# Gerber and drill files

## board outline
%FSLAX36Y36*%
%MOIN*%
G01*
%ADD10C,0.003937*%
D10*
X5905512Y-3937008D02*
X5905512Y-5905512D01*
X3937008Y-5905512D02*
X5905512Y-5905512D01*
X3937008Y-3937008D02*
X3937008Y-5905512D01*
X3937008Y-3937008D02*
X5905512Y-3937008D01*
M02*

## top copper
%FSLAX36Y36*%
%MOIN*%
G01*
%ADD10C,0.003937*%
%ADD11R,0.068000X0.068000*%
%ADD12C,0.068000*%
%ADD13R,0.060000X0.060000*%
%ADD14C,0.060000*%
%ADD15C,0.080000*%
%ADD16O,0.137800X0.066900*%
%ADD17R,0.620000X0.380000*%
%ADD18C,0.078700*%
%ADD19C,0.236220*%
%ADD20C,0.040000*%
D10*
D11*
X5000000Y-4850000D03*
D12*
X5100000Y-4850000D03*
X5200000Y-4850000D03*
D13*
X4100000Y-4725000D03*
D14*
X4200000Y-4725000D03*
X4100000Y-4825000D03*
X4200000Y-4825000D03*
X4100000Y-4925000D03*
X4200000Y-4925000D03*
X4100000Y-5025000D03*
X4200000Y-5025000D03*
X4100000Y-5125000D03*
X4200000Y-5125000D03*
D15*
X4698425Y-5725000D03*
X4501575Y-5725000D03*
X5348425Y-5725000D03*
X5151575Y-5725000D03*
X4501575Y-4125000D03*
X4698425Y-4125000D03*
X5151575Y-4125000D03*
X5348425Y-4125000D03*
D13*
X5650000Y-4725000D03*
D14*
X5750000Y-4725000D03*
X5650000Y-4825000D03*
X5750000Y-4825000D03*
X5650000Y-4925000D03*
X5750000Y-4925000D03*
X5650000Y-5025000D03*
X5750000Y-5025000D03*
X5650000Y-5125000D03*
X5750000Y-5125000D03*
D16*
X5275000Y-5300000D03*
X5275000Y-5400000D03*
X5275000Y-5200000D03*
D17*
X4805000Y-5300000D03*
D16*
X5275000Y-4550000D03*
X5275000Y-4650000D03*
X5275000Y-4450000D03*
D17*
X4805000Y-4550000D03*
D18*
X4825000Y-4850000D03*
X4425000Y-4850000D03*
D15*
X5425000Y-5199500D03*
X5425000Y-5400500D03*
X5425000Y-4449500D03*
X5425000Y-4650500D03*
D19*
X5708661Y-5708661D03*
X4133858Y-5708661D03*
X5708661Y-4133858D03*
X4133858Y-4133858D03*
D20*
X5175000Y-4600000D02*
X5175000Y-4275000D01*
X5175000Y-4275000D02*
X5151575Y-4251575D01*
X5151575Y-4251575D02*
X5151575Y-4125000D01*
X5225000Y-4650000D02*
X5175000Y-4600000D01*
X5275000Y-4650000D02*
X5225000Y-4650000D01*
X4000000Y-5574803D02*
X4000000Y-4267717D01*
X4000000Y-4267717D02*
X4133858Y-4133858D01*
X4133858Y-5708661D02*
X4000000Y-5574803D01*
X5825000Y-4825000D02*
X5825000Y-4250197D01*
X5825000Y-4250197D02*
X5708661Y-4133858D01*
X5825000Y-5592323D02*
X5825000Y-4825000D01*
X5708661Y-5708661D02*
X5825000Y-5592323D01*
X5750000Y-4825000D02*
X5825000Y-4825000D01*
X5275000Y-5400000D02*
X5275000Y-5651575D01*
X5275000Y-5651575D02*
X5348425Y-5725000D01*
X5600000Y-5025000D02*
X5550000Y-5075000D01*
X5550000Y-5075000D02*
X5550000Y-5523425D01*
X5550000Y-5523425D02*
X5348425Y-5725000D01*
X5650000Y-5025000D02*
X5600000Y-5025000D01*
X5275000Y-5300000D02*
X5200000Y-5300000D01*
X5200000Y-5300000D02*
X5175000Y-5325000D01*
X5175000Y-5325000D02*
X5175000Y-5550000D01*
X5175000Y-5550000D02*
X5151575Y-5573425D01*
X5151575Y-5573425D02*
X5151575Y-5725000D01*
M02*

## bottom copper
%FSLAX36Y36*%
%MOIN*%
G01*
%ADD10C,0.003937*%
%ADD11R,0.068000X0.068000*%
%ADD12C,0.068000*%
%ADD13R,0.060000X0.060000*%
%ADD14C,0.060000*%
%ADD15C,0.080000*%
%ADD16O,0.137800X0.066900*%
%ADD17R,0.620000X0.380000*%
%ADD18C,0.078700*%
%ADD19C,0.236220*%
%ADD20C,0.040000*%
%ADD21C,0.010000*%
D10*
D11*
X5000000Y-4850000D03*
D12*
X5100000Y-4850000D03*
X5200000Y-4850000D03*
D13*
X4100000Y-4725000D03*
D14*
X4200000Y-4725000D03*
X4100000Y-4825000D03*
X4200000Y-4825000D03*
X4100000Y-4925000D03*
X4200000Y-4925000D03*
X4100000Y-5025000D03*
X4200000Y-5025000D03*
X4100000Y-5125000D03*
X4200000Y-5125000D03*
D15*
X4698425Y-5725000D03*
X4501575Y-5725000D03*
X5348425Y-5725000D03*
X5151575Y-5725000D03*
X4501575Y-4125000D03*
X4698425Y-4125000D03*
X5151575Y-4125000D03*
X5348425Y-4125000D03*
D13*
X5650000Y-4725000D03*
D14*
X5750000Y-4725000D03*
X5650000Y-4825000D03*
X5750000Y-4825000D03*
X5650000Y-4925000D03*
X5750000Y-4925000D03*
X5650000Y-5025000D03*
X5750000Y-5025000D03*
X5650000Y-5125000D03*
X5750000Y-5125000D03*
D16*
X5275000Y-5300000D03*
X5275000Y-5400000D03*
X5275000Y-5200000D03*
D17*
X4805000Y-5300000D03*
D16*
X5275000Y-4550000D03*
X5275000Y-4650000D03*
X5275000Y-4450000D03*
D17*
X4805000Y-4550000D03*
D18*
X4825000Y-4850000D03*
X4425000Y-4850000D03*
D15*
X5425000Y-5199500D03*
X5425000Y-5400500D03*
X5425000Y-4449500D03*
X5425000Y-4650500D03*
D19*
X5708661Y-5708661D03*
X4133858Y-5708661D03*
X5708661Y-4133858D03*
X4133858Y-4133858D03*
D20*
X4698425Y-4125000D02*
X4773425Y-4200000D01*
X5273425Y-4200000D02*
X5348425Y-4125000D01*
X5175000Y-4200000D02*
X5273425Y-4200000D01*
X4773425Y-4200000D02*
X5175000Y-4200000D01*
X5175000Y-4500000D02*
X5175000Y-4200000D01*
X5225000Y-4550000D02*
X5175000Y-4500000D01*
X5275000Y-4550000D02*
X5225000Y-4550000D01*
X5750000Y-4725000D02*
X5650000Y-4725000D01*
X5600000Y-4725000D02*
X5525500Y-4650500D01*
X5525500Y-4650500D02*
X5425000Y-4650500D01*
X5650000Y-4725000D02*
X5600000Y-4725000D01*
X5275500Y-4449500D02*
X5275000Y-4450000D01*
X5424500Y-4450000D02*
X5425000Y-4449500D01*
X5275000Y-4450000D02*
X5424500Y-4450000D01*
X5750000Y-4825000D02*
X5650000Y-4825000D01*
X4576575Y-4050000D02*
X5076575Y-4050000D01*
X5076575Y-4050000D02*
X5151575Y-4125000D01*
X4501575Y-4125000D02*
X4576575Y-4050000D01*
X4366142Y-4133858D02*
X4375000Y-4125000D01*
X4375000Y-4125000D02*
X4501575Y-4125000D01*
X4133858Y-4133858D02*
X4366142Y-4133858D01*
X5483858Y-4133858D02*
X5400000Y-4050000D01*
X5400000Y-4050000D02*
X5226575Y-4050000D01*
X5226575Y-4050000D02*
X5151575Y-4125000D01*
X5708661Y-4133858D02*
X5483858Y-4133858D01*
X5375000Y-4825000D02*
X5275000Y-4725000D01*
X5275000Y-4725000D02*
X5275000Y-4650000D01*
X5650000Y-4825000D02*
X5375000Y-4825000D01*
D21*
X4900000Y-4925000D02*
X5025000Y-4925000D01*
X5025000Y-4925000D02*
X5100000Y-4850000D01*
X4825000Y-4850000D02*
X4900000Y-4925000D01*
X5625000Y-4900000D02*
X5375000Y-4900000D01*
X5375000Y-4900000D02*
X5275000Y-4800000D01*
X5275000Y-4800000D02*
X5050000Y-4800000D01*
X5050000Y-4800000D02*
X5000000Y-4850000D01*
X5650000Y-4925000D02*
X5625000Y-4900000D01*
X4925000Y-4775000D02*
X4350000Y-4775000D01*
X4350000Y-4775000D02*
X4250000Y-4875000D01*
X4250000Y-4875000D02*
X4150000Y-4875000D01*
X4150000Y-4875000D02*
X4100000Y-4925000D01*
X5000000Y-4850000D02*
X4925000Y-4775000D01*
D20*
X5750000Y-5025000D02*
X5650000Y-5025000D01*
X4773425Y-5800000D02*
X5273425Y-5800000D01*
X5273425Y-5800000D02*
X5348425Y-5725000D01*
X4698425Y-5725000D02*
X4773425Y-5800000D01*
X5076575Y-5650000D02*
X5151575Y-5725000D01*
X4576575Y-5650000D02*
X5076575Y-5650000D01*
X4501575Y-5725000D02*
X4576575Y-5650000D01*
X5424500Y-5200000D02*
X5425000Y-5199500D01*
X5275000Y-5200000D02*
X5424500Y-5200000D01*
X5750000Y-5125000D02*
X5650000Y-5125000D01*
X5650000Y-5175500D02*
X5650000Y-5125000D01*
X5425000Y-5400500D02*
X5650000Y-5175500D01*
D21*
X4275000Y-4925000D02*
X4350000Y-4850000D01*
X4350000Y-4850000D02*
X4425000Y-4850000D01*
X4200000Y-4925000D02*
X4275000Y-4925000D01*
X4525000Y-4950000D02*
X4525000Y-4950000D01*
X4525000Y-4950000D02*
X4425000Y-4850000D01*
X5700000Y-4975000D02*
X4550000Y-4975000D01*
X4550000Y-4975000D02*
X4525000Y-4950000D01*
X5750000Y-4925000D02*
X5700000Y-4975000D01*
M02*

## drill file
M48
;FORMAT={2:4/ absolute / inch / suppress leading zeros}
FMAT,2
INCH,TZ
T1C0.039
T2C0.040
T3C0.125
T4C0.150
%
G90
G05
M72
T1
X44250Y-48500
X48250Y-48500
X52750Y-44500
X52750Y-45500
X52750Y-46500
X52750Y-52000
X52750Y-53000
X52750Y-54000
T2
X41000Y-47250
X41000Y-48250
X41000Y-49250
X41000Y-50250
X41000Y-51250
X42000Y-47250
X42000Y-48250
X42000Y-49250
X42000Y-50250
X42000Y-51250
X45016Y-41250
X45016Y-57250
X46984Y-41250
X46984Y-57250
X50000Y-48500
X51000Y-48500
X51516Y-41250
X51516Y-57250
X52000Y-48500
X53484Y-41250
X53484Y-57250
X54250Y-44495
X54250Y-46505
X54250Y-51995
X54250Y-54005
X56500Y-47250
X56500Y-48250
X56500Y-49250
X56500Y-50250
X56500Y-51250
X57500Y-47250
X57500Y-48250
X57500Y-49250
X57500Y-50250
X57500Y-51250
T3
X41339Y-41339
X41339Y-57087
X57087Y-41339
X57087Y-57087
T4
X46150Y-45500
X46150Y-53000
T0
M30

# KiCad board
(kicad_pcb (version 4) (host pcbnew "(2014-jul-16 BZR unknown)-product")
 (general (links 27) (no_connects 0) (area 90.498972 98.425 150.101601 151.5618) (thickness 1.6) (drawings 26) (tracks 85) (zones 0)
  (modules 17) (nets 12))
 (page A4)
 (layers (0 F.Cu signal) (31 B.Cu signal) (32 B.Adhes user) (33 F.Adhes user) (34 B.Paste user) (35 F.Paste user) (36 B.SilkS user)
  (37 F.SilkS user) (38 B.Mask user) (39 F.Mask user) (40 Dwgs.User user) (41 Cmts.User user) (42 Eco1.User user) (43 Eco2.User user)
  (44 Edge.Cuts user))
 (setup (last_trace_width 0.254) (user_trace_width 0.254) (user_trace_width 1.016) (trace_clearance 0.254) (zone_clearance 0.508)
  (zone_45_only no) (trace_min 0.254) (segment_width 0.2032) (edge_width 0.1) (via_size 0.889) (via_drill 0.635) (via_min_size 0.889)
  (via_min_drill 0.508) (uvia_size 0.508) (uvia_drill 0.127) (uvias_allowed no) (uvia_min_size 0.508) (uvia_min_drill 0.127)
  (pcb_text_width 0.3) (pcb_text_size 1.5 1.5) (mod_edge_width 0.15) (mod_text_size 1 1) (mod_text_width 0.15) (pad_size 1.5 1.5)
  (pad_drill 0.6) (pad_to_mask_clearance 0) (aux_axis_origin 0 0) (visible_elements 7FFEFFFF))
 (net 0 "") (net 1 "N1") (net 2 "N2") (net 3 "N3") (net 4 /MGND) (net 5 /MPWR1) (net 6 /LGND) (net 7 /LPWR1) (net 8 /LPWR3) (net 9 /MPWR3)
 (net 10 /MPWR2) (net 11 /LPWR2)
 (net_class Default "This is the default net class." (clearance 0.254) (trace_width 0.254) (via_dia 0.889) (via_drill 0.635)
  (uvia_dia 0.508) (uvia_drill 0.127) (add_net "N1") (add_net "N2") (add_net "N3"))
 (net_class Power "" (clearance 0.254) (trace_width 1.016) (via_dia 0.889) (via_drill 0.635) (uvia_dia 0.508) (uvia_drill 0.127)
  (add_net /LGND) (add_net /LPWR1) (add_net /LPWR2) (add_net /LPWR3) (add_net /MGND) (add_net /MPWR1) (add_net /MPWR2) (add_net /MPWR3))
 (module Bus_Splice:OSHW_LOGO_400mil (layer B.Cu) (at 125.73 113.03 180)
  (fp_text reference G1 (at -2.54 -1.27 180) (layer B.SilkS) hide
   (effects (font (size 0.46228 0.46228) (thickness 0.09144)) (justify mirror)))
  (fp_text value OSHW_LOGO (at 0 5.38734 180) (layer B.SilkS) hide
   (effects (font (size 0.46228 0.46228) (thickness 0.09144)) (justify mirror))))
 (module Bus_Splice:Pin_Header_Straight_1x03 (layer F.Cu) (at 129.54 123.19)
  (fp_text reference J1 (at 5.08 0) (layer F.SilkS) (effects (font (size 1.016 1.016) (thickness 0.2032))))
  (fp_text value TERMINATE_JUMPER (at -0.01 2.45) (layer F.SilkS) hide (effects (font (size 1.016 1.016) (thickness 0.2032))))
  (pad 1 thru_hole rect (at -2.54 0) (size 1.7272 1.7272) (drill 1.016) (layers *.Cu *.Mask F.SilkS) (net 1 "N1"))
  (pad 2 thru_hole circle (at 0 0) (size 1.7272 1.7272) (drill 1.016) (layers *.Cu *.Mask F.SilkS) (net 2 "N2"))
  (pad 3 thru_hole circle (at 2.54 0) (size 1.7272 1.7272) (drill 1.016) (layers *.Cu *.Mask F.SilkS)))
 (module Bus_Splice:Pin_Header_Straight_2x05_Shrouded (layer F.Cu) (at 105.41 125.095 270)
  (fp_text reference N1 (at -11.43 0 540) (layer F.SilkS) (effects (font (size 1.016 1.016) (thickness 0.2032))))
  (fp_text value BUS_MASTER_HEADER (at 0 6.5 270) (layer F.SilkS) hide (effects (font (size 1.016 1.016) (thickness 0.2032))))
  (pad 1 thru_hole rect (at -5.08 1.27 270) (size 1.524 1.524) (drill 1.016) (layers *.Cu *.Mask F.SilkS))
  (pad 2 thru_hole circle (at -5.08 -1.27 270) (size 1.524 1.524) (drill 1.016) (layers *.Cu *.Mask F.SilkS))
  (pad 3 thru_hole circle (at -2.54 1.27 270) (size 1.524 1.524) (drill 1.016) (layers *.Cu *.Mask F.SilkS))
  (pad 4 thru_hole circle (at -2.54 -1.27 270) (size 1.524 1.524) (drill 1.016) (layers *.Cu *.Mask F.SilkS))
  (pad 5 thru_hole circle (at 0 1.27 270) (size 1.524 1.524) (drill 1.016) (layers *.Cu *.Mask F.SilkS) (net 1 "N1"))
  (pad 6 thru_hole circle (at 0 -1.27 270) (size 1.524 1.524) (drill 1.016) (layers *.Cu *.Mask F.SilkS) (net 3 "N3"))
  (pad 7 thru_hole circle (at 2.54 1.27 270) (size 1.524 1.524) (drill 1.016) (layers *.Cu *.Mask F.SilkS))
  (pad 8 thru_hole circle (at 2.54 -1.27 270) (size 1.524 1.524) (drill 1.016) (layers *.Cu *.Mask F.SilkS))
  (pad 9 thru_hole circle (at 5.08 1.27 270) (size 1.524 1.524) (drill 1.016) (layers *.Cu *.Mask F.SilkS))
  (pad 10 thru_hole circle (at 5.08 -1.27 270) (size 1.524 1.524) (drill 1.016) (layers *.Cu *.Mask F.SilkS)))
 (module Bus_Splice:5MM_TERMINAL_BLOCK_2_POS (layer F.Cu) (at 116.84 145.415 180)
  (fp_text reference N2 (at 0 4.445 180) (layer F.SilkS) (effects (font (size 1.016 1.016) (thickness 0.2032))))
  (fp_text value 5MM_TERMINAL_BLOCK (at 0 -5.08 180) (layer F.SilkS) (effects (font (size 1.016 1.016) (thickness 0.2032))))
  (pad 1 thru_hole circle (at -2.5 0 180) (size 2.032 2.032) (drill 1.016) (layers *.Cu *.Mask) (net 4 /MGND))
  (pad 2 thru_hole circle (at 2.5 0 180) (size 2.032 2.032) (drill 1.016) (layers *.Cu *.Mask) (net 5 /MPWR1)))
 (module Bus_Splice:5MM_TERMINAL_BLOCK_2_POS (layer F.Cu) (at 133.35 145.415 180)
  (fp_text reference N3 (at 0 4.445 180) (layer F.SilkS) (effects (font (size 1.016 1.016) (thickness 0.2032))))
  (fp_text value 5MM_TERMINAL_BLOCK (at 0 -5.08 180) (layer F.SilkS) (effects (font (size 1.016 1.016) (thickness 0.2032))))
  (pad 1 thru_hole circle (at -2.5 0 180) (size 2.032 2.032) (drill 1.016) (layers *.Cu *.Mask) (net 4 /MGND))
  (pad 2 thru_hole circle (at 2.5 0 180) (size 2.032 2.032) (drill 1.016) (layers *.Cu *.Mask) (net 5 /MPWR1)))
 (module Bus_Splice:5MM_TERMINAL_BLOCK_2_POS (layer F.Cu) (at 116.84 104.775)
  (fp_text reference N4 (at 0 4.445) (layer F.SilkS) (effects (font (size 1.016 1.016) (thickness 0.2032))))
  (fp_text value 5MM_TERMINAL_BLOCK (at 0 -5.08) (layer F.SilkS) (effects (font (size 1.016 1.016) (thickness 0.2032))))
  (pad 1 thru_hole circle (at -2.5 0) (size 2.032 2.032) (drill 1.016) (layers *.Cu *.Mask) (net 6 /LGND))
  (pad 2 thru_hole circle (at 2.5 0) (size 2.032 2.032) (drill 1.016) (layers *.Cu *.Mask) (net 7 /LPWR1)))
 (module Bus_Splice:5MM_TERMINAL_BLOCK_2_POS (layer F.Cu) (at 133.35 104.775)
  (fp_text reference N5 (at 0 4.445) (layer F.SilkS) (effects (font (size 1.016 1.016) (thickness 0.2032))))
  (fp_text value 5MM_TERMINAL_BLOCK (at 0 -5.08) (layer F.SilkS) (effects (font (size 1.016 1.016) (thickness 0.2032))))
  (pad 1 thru_hole circle (at -2.5 0) (size 2.032 2.032) (drill 1.016) (layers *.Cu *.Mask) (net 6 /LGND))
  (pad 2 thru_hole circle (at 2.5 0) (size 2.032 2.032) (drill 1.016) (layers *.Cu *.Mask) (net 7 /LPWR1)))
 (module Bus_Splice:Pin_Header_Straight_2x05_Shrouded (layer F.Cu) (at 144.78 125.095 270)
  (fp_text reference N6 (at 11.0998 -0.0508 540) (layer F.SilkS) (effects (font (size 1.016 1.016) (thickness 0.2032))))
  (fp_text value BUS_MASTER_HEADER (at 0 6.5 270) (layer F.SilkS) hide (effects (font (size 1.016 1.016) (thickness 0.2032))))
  (pad 1 thru_hole rect (at -5.08 1.27 270) (size 1.524 1.524) (drill 1.016) (layers *.Cu *.Mask F.SilkS) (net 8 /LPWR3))
  (pad 2 thru_hole circle (at -5.08 -1.27 270) (size 1.524 1.524) (drill 1.016) (layers *.Cu *.Mask F.SilkS) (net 8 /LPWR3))
  (pad 3 thru_hole circle (at -2.54 1.27 270) (size 1.524 1.524) (drill 1.016) (layers *.Cu *.Mask F.SilkS) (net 6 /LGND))
  (pad 4 thru_hole circle (at -2.54 -1.27 270) (size 1.524 1.524) (drill 1.016) (layers *.Cu *.Mask F.SilkS) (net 6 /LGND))
  (pad 5 thru_hole circle (at 0 1.27 270) (size 1.524 1.524) (drill 1.016) (layers *.Cu *.Mask F.SilkS) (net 1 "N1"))
  (pad 6 thru_hole circle (at 0 -1.27 270) (size 1.524 1.524) (drill 1.016) (layers *.Cu *.Mask F.SilkS) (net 3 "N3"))
  (pad 7 thru_hole circle (at 2.54 1.27 270) (size 1.524 1.524) (drill 1.016) (layers *.Cu *.Mask F.SilkS) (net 4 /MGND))
  (pad 8 thru_hole circle (at 2.54 -1.27 270) (size 1.524 1.524) (drill 1.016) (layers *.Cu *.Mask F.SilkS) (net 4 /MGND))
  (pad 9 thru_hole circle (at 5.08 1.27 270) (size 1.524 1.524) (drill 1.016) (layers *.Cu *.Mask F.SilkS) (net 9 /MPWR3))
  (pad 10 thru_hole circle (at 5.08 -1.27 270) (size 1.524 1.524) (drill 1.016) (layers *.Cu *.Mask F.SilkS) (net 9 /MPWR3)))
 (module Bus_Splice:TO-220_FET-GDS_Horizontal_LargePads (layer F.Cu) (at 133.985 134.62 90)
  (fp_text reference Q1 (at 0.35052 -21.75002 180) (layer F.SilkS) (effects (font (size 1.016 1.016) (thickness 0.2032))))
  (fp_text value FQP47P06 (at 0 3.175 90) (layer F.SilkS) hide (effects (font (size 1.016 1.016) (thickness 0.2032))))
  (pad D thru_hole oval (at 0 0 180) (size 3.50012 1.69926) (drill 1.00076) (layers *.Cu *.Mask F.SilkS) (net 5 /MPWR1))
  (pad G thru_hole oval (at -2.54 0 180) (size 3.50012 1.69926) (drill 1.00076) (layers *.Cu *.Mask F.SilkS) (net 4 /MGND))
  (pad S thru_hole oval (at 2.54 0 180) (size 3.50012 1.69926) (drill 1.00076) (layers *.Cu *.Mask F.SilkS) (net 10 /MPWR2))
  (pad 2 thru_hole rect (at 0 -16.764 180) (size 15.748 9.652) (drill 3.79984 (offset -4.826 0)) (layers *.Cu F.SilkS F.Mask)))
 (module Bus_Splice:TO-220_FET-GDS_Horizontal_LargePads (layer F.Cu) (at 133.985 115.57 90)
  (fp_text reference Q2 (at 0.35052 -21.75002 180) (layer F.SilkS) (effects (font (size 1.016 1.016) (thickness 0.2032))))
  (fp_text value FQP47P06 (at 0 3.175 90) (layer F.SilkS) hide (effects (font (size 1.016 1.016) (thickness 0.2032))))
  (pad D thru_hole oval (at 0 0 180) (size 3.50012 1.69926) (drill 1.00076) (layers *.Cu *.Mask F.SilkS) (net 7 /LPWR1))
  (pad G thru_hole oval (at -2.54 0 180) (size 3.50012 1.69926) (drill 1.00076) (layers *.Cu *.Mask F.SilkS) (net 6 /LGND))
  (pad S thru_hole oval (at 2.54 0 180) (size 3.50012 1.69926) (drill 1.00076) (layers *.Cu *.Mask F.SilkS) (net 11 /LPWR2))
  (pad 2 thru_hole rect (at 0 -16.764 180) (size 15.748 9.652) (drill 3.79984 (offset -4.826 0)) (layers *.Cu F.SilkS F.Mask)))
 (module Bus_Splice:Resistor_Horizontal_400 (layer F.Cu) (at 117.475 123.19 180)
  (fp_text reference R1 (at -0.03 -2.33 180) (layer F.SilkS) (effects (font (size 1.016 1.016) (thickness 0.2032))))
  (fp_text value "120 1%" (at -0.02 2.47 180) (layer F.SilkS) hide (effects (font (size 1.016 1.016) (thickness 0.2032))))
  (pad 1 thru_hole circle (at -5.08 0 180) (size 1.99898 1.99898) (drill 1.00076) (layers *.Cu *.SilkS *.Mask) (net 2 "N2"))
  (pad 2 thru_hole circle (at 5.08 0 180) (size 1.99898 1.99898) (drill 1.00076) (layers *.Cu *.SilkS *.Mask) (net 3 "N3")))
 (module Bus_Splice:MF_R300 (layer F.Cu) (at 137.795 134.62 270)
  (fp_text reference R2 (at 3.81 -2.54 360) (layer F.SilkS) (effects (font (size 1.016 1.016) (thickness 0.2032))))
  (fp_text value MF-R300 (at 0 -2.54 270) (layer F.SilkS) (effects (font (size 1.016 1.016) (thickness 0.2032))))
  (pad 1 thru_hole circle (at -2.5527 0 270) (size 2.032 2.032) (drill 1.016) (layers *.Cu *.Mask) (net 10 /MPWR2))
  (pad 2 thru_hole circle (at 2.5527 0 270) (size 2.032 2.032) (drill 1.016) (layers *.Cu *.Mask) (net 9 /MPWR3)))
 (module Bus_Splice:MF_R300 (layer F.Cu) (at 137.795 115.57 270)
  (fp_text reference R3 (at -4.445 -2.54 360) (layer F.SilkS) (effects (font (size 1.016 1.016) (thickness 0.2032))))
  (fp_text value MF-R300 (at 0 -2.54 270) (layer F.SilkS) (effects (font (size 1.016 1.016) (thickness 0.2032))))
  (pad 1 thru_hole circle (at -2.5527 0 270) (size 2.032 2.032) (drill 1.016) (layers *.Cu *.Mask) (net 11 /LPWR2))
  (pad 2 thru_hole circle (at 2.5527 0 270) (size 2.032 2.032) (drill 1.016) (layers *.Cu *.Mask) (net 8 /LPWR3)))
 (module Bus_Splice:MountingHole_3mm (layer F.Cu) (at 145 145)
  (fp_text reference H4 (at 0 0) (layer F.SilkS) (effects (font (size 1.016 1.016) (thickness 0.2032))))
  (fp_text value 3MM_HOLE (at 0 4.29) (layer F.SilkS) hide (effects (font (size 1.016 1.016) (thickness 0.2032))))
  (pad 1 thru_hole circle (at 0 0) (size 6 6) (drill 3.175) (layers *.Cu *.SilkS *.Mask) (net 6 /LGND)))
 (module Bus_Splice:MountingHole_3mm (layer F.Cu) (at 105 145)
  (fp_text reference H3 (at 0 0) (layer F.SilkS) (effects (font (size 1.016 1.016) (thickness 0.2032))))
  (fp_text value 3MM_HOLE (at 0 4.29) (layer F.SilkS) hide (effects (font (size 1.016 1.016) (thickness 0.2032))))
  (pad 1 thru_hole circle (at 0 0) (size 6 6) (drill 3.175) (layers *.Cu *.SilkS *.Mask) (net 6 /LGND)))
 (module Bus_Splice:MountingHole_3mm (layer F.Cu) (at 145 105)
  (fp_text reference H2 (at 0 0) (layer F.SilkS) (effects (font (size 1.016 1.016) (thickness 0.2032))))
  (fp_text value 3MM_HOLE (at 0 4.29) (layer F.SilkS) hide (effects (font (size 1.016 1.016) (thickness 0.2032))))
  (pad 1 thru_hole circle (at 0 0) (size 6 6) (drill 3.175) (layers *.Cu *.SilkS *.Mask) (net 6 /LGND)))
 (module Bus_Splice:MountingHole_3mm (layer F.Cu) (at 105 105)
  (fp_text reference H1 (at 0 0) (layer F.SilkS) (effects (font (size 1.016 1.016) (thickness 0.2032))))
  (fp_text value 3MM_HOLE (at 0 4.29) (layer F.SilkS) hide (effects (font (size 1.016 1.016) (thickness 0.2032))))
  (pad 1 thru_hole circle (at 0 0) (size 6 6) (drill 3.175) (layers *.Cu *.SilkS *.Mask) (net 6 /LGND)))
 (gr_line (start 150 100) (end 150 150) (angle 90) (layer Edge.Cuts) (width 0.1))
 (gr_line (start 100 150) (end 150 150) (angle 90) (layer Edge.Cuts) (width 0.1))
 (gr_line (start 100 100) (end 100 150) (angle 90) (layer Edge.Cuts) (width 0.1))
 (gr_line (start 100 100) (end 150 100) (angle 90) (layer Edge.Cuts) (width 0.1))
 (segment (start 119.34 104.775) (end 121.245 106.68) (width 1.016) (layer B.Cu) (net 7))
 (segment (start 133.945 106.68) (end 135.85 104.775) (width 1.016) (layer B.Cu) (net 7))
 (segment (start 131.445 106.68) (end 133.945 106.68) (width 1.016) (layer B.Cu) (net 7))
 (segment (start 121.245 106.68) (end 131.445 106.68) (width 1.016) (layer B.Cu) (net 7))
 (segment (start 131.445 114.3) (end 131.445 106.68) (width 1.016) (layer B.Cu) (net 7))
 (segment (start 132.715 115.57) (end 131.445 114.3) (width 1.016) (layer B.Cu) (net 7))
 (segment (start 133.985 115.57) (end 132.715 115.57) (width 1.016) (layer B.Cu) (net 7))
 (segment (start 146.05 120.015) (end 143.51 120.015) (width 1.016) (layer B.Cu) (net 8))
 (segment (start 142.24 120.015) (end 140.3477 118.1227) (width 1.016) (layer B.Cu) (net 8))
 (segment (start 140.3477 118.1227) (end 137.795 118.1227) (width 1.016) (layer B.Cu) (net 8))
 (segment (start 143.51 120.015) (end 142.24 120.015) (width 1.016) (layer B.Cu) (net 8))
 (segment (start 133.9977 113.0173) (end 133.985 113.03) (width 1.016) (layer B.Cu) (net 11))
 (segment (start 137.7823 113.03) (end 137.795 113.0173) (width 1.016) (layer B.Cu) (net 11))
 (segment (start 133.985 113.03) (end 137.7823 113.03) (width 1.016) (layer B.Cu) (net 11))
 (segment (start 131.445 116.84) (end 131.445 108.585) (width 1.016) (layer F.Cu) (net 6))
 (segment (start 131.445 108.585) (end 130.85 107.99) (width 1.016) (layer F.Cu) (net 6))
 (segment (start 130.85 107.99) (end 130.85 104.775) (width 1.016) (layer F.Cu) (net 6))
 (segment (start 132.715 118.11) (end 131.445 116.84) (width 1.016) (layer F.Cu) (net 6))
 (segment (start 133.985 118.11) (end 132.715 118.11) (width 1.016) (layer F.Cu) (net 6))
 (segment (start 146.05 122.555) (end 143.51 122.555) (width 1.016) (layer B.Cu) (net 6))
 (segment (start 101.6 141.6) (end 101.6 108.4) (width 1.016) (layer F.Cu) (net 6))
 (segment (start 101.6 108.4) (end 105 105) (width 1.016) (layer F.Cu) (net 6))
 (segment (start 105 145) (end 101.6 141.6) (width 1.016) (layer F.Cu) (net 6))
 (segment (start 116.245 102.87) (end 128.945 102.87) (width 1.016) (layer B.Cu) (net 6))
 (segment (start 128.945 102.87) (end 130.85 104.775) (width 1.016) (layer B.Cu) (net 6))
 (segment (start 114.34 104.775) (end 116.245 102.87) (width 1.016) (layer B.Cu) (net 6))
 (segment (start 110.9 105) (end 111.125 104.775) (width 1.016) (layer B.Cu) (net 6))
 (segment (start 111.125 104.775) (end 114.34 104.775) (width 1.016) (layer B.Cu) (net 6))
 (segment (start 105 105) (end 110.9 105) (width 1.016) (layer B.Cu) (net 6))
 (segment (start 139.29 105) (end 137.16 102.87) (width 1.016) (layer B.Cu) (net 6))
 (segment (start 137.16 102.87) (end 132.755 102.87) (width 1.016) (layer B.Cu) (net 6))
 (segment (start 132.755 102.87) (end 130.85 104.775) (width 1.016) (layer B.Cu) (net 6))
 (segment (start 145 105) (end 139.29 105) (width 1.016) (layer B.Cu) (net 6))
 (segment (start 136.525 122.555) (end 133.985 120.015) (width 1.016) (layer B.Cu) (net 6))
 (segment (start 133.985 120.015) (end 133.985 118.11) (width 1.016) (layer B.Cu) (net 6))
 (segment (start 143.51 122.555) (end 136.525 122.555) (width 1.016) (layer B.Cu) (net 6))
 (segment (start 147.955 122.555) (end 147.955 107.955) (width 1.016) (layer F.Cu) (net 6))
 (segment (start 147.955 107.955) (end 145 105) (width 1.016) (layer F.Cu) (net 6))
 (segment (start 147.955 142.045) (end 147.955 122.555) (width 1.016) (layer F.Cu) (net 6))
 (segment (start 145 145) (end 147.955 142.045) (width 1.016) (layer F.Cu) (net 6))
 (segment (start 146.05 122.555) (end 147.955 122.555) (width 1.016) (layer F.Cu) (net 6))
 (segment (start 124.46 125.095) (end 127.635 125.095) (width 0.254) (layer B.Cu) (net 2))
 (segment (start 127.635 125.095) (end 129.54 123.19) (width 0.254) (layer B.Cu) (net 2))
 (segment (start 122.555 123.19) (end 124.46 125.095) (width 0.254) (layer B.Cu) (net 2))
 (segment (start 142.875 124.46) (end 136.525 124.46) (width 0.254) (layer B.Cu) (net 1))
 (segment (start 136.525 124.46) (end 133.985 121.92) (width 0.254) (layer B.Cu) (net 1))
 (segment (start 133.985 121.92) (end 128.27 121.92) (width 0.254) (layer B.Cu) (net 1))
 (segment (start 128.27 121.92) (end 127 123.19) (width 0.254) (layer B.Cu) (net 1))
 (segment (start 143.51 125.095) (end 142.875 124.46) (width 0.254) (layer B.Cu) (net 1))
 (segment (start 125.095 121.285) (end 110.49 121.285) (width 0.254) (layer B.Cu) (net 1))
 (segment (start 110.49 121.285) (end 107.95 123.825) (width 0.254) (layer B.Cu) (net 1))
 (segment (start 107.95 123.825) (end 105.41 123.825) (width 0.254) (layer B.Cu) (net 1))
 (segment (start 105.41 123.825) (end 104.14 125.095) (width 0.254) (layer B.Cu) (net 1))
 (segment (start 127 123.19) (end 125.095 121.285) (width 0.254) (layer B.Cu) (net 1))
 (segment (start 146.05 127.635) (end 143.51 127.635) (width 1.016) (layer B.Cu) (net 4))
 (segment (start 133.985 137.16) (end 133.985 143.55) (width 1.016) (layer F.Cu) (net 4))
 (segment (start 133.985 143.55) (end 135.85 145.415) (width 1.016) (layer F.Cu) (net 4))
 (segment (start 121.245 147.32) (end 133.945 147.32) (width 1.016) (layer B.Cu) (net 4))
 (segment (start 133.945 147.32) (end 135.85 145.415) (width 1.016) (layer B.Cu) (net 4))
 (segment (start 119.34 145.415) (end 121.245 147.32) (width 1.016) (layer B.Cu) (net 4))
 (segment (start 142.24 127.635) (end 140.97 128.905) (width 1.016) (layer F.Cu) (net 4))
 (segment (start 140.97 128.905) (end 140.97 140.295) (width 1.016) (layer F.Cu) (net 4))
 (segment (start 140.97 140.295) (end 135.85 145.415) (width 1.016) (layer F.Cu) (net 4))
 (segment (start 143.51 127.635) (end 142.24 127.635) (width 1.016) (layer F.Cu) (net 4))
 (segment (start 133.985 134.62) (end 132.08 134.62) (width 1.016) (layer F.Cu) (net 5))
 (segment (start 132.08 134.62) (end 131.445 135.255) (width 1.016) (layer F.Cu) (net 5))
 (segment (start 131.445 135.255) (end 131.445 140.97) (width 1.016) (layer F.Cu) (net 5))
 (segment (start 131.445 140.97) (end 130.85 141.565) (width 1.016) (layer F.Cu) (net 5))
 (segment (start 130.85 141.565) (end 130.85 145.415) (width 1.016) (layer F.Cu) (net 5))
 (segment (start 128.945 143.51) (end 130.85 145.415) (width 1.016) (layer B.Cu) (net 5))
 (segment (start 116.245 143.51) (end 128.945 143.51) (width 1.016) (layer B.Cu) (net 5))
 (segment (start 114.34 145.415) (end 116.245 143.51) (width 1.016) (layer B.Cu) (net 5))
 (segment (start 137.7823 132.08) (end 137.795 132.0673) (width 1.016) (layer B.Cu) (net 10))
 (segment (start 133.985 132.08) (end 137.7823 132.08) (width 1.016) (layer B.Cu) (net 10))
 (segment (start 146.05 130.175) (end 143.51 130.175) (width 1.016) (layer B.Cu) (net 9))
 (segment (start 143.51 131.4577) (end 143.51 130.175) (width 1.016) (layer B.Cu) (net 9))
 (segment (start 137.795 137.1727) (end 143.51 131.4577) (width 1.016) (layer B.Cu) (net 9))
 (segment (start 108.585 125.095) (end 110.49 123.19) (width 0.254) (layer B.Cu) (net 3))
 (segment (start 110.49 123.19) (end 112.395 123.19) (width 0.254) (layer B.Cu) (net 3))
 (segment (start 106.68 125.095) (end 108.585 125.095) (width 0.254) (layer B.Cu) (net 3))
 (segment (start 114.935 125.73) (end 114.935 125.73) (width 0.254) (layer B.Cu) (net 3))
 (segment (start 114.935 125.73) (end 112.395 123.19) (width 0.254) (layer B.Cu) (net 3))
 (segment (start 144.78 126.365) (end 115.57 126.365) (width 0.254) (layer B.Cu) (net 3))
 (segment (start 115.57 126.365) (end 114.935 125.73) (width 0.254) (layer B.Cu) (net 3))
 (segment (start 146.05 125.095) (end 144.78 126.365) (width 0.254) (layer B.Cu) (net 3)))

